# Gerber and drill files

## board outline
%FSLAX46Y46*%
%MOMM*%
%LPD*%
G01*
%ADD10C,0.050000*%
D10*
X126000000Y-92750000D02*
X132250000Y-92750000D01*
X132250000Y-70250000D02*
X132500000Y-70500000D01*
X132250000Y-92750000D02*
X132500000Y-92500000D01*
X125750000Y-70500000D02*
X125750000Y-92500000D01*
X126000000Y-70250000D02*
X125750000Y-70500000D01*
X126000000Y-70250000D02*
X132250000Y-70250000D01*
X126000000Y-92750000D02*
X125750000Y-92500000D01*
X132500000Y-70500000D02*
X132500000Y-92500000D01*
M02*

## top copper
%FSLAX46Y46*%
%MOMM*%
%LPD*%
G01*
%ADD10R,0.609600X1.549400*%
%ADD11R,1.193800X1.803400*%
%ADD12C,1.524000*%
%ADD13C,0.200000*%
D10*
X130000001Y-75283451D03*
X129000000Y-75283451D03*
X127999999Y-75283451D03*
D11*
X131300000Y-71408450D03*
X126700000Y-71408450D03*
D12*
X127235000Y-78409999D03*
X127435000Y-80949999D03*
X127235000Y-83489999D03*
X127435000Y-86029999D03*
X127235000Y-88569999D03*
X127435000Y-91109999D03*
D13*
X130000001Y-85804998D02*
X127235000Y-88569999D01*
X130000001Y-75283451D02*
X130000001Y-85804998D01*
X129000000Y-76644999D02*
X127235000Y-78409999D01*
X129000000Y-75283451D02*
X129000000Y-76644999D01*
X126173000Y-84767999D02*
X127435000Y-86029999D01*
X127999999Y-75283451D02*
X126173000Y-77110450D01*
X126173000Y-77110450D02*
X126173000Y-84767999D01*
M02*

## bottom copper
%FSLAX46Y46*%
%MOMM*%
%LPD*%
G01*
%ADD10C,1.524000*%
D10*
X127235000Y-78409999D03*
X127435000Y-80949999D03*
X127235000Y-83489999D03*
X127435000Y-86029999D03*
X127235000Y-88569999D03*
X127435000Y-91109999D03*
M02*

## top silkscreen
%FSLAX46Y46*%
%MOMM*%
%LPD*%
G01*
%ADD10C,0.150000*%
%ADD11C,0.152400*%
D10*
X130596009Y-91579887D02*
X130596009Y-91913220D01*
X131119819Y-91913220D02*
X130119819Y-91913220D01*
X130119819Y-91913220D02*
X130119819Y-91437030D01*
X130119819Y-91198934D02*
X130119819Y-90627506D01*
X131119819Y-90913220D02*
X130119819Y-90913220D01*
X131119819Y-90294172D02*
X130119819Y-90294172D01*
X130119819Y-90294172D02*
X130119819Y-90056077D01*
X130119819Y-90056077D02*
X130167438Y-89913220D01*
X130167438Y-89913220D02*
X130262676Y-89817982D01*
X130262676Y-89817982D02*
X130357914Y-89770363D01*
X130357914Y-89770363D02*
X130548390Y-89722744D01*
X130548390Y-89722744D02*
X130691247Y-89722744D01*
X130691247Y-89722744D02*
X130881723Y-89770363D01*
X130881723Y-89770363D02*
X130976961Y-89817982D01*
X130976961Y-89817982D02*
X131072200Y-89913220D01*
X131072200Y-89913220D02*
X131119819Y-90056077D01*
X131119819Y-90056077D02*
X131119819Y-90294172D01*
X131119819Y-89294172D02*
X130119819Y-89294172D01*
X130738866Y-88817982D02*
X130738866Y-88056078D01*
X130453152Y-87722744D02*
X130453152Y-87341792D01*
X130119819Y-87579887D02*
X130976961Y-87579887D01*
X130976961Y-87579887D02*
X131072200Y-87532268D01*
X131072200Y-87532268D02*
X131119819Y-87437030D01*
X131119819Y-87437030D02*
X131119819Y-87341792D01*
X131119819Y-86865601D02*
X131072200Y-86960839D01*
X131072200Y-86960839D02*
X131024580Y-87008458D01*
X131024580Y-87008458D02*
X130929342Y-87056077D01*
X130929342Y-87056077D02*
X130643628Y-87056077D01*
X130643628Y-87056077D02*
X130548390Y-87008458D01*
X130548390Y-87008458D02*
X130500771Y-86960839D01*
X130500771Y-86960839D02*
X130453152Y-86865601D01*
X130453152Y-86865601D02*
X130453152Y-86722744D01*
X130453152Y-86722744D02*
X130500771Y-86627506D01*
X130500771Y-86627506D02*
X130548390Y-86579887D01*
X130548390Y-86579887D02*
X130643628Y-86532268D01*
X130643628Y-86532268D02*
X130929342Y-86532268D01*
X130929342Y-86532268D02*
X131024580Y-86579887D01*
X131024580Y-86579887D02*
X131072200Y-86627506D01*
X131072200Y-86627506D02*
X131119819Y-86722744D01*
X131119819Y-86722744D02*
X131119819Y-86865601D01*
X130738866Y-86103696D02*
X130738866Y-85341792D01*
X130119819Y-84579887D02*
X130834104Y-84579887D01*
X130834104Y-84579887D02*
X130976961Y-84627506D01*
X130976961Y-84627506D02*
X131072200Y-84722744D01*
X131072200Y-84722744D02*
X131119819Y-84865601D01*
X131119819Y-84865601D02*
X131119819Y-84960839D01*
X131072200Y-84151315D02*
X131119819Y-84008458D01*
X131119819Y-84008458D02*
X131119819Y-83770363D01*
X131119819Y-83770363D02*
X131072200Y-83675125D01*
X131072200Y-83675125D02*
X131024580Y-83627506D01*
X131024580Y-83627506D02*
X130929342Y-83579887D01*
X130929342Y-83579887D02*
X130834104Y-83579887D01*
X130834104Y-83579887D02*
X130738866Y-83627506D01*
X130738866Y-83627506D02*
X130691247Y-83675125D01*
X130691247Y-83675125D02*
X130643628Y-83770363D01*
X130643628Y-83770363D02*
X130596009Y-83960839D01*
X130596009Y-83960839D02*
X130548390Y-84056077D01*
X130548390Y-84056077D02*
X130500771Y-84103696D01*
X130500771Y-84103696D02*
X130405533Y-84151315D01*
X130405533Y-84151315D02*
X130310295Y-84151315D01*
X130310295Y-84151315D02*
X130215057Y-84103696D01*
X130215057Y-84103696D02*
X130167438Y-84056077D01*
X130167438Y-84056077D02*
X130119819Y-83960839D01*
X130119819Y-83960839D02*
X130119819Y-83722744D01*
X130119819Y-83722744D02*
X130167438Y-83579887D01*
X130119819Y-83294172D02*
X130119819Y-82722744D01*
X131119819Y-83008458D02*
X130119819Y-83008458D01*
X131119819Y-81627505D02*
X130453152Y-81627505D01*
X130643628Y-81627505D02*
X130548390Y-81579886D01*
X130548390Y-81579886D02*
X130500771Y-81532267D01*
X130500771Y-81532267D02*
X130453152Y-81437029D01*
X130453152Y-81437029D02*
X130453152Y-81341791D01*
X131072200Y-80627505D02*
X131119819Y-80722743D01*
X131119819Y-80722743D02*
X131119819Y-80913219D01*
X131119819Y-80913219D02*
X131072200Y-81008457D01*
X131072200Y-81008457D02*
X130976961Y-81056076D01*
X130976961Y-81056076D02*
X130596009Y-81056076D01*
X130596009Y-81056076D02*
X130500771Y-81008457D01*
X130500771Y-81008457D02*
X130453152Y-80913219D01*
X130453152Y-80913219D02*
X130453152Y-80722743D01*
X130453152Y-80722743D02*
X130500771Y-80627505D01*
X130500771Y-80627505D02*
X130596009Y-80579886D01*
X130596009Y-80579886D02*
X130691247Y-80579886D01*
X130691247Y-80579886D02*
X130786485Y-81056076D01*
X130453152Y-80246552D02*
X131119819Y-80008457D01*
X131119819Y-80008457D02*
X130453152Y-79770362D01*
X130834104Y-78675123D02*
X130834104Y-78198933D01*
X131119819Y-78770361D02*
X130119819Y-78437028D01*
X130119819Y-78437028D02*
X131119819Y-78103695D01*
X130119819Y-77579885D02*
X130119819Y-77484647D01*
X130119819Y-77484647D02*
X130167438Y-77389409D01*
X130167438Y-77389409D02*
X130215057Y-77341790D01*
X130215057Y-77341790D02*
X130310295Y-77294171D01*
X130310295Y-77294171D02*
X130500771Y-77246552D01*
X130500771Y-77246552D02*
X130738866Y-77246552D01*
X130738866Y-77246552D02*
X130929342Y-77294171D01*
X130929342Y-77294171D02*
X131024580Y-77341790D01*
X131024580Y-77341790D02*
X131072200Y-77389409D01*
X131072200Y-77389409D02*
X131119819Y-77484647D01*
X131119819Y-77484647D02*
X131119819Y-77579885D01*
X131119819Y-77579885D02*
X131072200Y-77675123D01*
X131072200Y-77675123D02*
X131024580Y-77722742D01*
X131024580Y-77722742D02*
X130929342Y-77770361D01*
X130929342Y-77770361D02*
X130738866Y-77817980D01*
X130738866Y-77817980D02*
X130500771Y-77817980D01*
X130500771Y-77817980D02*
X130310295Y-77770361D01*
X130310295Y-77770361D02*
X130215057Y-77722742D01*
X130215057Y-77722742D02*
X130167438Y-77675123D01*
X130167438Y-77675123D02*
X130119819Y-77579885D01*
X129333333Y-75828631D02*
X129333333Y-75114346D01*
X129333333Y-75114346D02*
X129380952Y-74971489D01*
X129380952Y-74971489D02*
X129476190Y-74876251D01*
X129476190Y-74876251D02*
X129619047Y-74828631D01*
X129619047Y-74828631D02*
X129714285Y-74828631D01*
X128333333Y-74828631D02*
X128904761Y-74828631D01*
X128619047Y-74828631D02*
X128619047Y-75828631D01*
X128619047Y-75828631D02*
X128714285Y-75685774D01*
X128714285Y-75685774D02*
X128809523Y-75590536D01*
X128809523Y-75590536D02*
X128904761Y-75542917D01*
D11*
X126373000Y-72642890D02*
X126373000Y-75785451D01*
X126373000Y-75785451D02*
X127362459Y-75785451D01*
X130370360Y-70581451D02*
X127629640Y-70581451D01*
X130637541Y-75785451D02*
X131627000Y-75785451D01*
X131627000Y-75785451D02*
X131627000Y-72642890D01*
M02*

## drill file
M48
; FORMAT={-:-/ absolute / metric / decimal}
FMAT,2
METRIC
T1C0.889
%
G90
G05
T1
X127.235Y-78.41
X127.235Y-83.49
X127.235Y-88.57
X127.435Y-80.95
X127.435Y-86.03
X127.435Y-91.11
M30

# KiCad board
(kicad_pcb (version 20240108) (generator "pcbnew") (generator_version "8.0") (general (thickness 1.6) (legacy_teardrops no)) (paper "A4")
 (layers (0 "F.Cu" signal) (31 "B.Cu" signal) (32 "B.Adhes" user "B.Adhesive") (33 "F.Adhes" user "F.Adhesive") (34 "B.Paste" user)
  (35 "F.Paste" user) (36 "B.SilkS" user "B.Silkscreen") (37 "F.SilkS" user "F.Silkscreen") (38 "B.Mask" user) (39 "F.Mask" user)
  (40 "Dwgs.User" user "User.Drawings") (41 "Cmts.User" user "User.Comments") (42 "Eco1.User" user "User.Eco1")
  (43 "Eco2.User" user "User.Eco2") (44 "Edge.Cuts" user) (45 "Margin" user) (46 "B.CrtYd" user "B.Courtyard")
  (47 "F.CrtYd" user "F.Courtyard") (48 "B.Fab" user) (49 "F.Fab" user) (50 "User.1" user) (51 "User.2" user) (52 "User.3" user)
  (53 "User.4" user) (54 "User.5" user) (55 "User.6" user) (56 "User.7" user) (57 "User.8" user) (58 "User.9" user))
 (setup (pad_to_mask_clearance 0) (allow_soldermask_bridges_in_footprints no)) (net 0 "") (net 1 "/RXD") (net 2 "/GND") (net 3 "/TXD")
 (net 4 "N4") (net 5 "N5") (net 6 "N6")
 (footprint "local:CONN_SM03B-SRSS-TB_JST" (layer "F.Cu") (at 129 73.183451 180)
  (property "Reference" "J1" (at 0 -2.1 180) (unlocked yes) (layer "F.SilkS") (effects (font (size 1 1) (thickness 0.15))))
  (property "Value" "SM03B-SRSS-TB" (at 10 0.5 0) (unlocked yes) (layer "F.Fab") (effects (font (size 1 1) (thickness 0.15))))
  (fp_line (start 2.627 0.540561) (end 2.627 -2.602) (stroke (width 0.1524) (type solid)) (layer "F.SilkS"))
  (fp_line (start 2.627 -2.602) (end 1.637541 -2.602) (stroke (width 0.1524) (type solid)) (layer "F.SilkS"))
  (fp_line (start -1.37036 2.602) (end 1.37036 2.602) (stroke (width 0.1524) (type solid)) (layer "F.SilkS"))
  (fp_line (start -1.637541 -2.602) (end -2.627 -2.602) (stroke (width 0.1524) (type solid)) (layer "F.SilkS"))
  (fp_line (start -2.627 -2.602) (end -2.627 0.540561) (stroke (width 0.1524) (type solid)) (layer "F.SilkS"))
  (pad "1" smd rect (at -1.000001 -2.1 180) (size 0.6096 1.5494) (layers "F.Cu" "F.Paste" "F.Mask") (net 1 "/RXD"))
  (pad "2" smd rect (at 0 -2.1 180) (size 0.6096 1.5494) (layers "F.Cu" "F.Paste" "F.Mask") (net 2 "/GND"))
  (pad "3" smd rect (at 1.000001 -2.1 180) (size 0.6096 1.5494) (layers "F.Cu" "F.Paste" "F.Mask") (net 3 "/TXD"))
  (pad "4" smd rect (at -2.3 1.775001 180) (size 1.1938 1.8034) (layers "F.Cu" "F.Paste" "F.Mask"))
  (pad "5" smd rect (at 2.3 1.775001 180) (size 1.1938 1.8034) (layers "F.Cu" "F.Paste" "F.Mask")))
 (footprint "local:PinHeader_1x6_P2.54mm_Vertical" (layer "F.Cu") (at 127.535 78.384999)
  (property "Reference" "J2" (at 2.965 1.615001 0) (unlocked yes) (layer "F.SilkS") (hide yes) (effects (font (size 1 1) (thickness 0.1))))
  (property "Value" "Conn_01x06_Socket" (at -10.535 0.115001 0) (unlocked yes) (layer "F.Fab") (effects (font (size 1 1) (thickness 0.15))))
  (pad "1" thru_hole circle (at -0.3 0.025) (size 1.524 1.524) (drill 0.889) (layers "*.Cu" "*.Mask") (remove_unused_layers no)
   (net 2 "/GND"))
  (pad "2" thru_hole circle (at -0.1 2.565) (size 1.524 1.524) (drill 0.889) (layers "*.Cu" "*.Mask") (remove_unused_layers no) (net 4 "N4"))
  (pad "3" thru_hole circle (at -0.3 5.105) (size 1.524 1.524) (drill 0.889) (layers "*.Cu" "*.Mask") (remove_unused_layers no) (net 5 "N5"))
  (pad "4" thru_hole circle (at -0.1 7.645) (size 1.524 1.524) (drill 0.889) (layers "*.Cu" "*.Mask") (remove_unused_layers no)
   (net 3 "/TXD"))
  (pad "5" thru_hole circle (at -0.3 10.185) (size 1.524 1.524) (drill 0.889) (layers "*.Cu" "*.Mask") (remove_unused_layers no)
   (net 1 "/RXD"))
  (pad "6" thru_hole circle (at -0.1 12.725) (size 1.524 1.524) (drill 0.889) (layers "*.Cu" "*.Mask") (remove_unused_layers no)
   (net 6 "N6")))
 (gr_line (start 126 92.75) (end 132.25 92.75) (stroke (width 0.05) (type default)) (layer "Edge.Cuts"))
 (gr_line (start 132.25 70.25) (end 132.5 70.5) (stroke (width 0.05) (type default)) (layer "Edge.Cuts"))
 (gr_line (start 132.25 92.75) (end 132.5 92.5) (stroke (width 0.05) (type default)) (layer "Edge.Cuts"))
 (gr_line (start 125.75 70.5) (end 125.75 92.5) (stroke (width 0.05) (type default)) (layer "Edge.Cuts"))
 (gr_line (start 126 70.25) (end 125.75 70.5) (stroke (width 0.05) (type default)) (layer "Edge.Cuts"))
 (gr_line (start 126 70.25) (end 132.25 70.25) (stroke (width 0.05) (type default)) (layer "Edge.Cuts"))
 (gr_line (start 126 92.75) (end 125.75 92.5) (stroke (width 0.05) (type default)) (layer "Edge.Cuts"))
 (gr_line (start 132.5 70.5) (end 132.5 92.5) (stroke (width 0.05) (type default)) (layer "Edge.Cuts"))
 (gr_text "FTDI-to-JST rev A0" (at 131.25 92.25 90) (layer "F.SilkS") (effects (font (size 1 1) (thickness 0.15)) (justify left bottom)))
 (segment (start 130.000001 85.804998) (end 127.235 88.569999) (width 0.2) (layer "F.Cu") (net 1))
 (segment (start 130.000001 75.283451) (end 130.000001 85.804998) (width 0.2) (layer "F.Cu") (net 1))
 (segment (start 129 76.644999) (end 127.235 78.409999) (width 0.2) (layer "F.Cu") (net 2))
 (segment (start 129 75.283451) (end 129 76.644999) (width 0.2) (layer "F.Cu") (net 2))
 (segment (start 126.173 84.767999) (end 127.435 86.029999) (width 0.2) (layer "F.Cu") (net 3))
 (segment (start 127.999999 75.283451) (end 126.173 77.11045) (width 0.2) (layer "F.Cu") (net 3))
 (segment (start 126.173 77.11045) (end 126.173 84.767999) (width 0.2) (layer "F.Cu") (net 3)))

